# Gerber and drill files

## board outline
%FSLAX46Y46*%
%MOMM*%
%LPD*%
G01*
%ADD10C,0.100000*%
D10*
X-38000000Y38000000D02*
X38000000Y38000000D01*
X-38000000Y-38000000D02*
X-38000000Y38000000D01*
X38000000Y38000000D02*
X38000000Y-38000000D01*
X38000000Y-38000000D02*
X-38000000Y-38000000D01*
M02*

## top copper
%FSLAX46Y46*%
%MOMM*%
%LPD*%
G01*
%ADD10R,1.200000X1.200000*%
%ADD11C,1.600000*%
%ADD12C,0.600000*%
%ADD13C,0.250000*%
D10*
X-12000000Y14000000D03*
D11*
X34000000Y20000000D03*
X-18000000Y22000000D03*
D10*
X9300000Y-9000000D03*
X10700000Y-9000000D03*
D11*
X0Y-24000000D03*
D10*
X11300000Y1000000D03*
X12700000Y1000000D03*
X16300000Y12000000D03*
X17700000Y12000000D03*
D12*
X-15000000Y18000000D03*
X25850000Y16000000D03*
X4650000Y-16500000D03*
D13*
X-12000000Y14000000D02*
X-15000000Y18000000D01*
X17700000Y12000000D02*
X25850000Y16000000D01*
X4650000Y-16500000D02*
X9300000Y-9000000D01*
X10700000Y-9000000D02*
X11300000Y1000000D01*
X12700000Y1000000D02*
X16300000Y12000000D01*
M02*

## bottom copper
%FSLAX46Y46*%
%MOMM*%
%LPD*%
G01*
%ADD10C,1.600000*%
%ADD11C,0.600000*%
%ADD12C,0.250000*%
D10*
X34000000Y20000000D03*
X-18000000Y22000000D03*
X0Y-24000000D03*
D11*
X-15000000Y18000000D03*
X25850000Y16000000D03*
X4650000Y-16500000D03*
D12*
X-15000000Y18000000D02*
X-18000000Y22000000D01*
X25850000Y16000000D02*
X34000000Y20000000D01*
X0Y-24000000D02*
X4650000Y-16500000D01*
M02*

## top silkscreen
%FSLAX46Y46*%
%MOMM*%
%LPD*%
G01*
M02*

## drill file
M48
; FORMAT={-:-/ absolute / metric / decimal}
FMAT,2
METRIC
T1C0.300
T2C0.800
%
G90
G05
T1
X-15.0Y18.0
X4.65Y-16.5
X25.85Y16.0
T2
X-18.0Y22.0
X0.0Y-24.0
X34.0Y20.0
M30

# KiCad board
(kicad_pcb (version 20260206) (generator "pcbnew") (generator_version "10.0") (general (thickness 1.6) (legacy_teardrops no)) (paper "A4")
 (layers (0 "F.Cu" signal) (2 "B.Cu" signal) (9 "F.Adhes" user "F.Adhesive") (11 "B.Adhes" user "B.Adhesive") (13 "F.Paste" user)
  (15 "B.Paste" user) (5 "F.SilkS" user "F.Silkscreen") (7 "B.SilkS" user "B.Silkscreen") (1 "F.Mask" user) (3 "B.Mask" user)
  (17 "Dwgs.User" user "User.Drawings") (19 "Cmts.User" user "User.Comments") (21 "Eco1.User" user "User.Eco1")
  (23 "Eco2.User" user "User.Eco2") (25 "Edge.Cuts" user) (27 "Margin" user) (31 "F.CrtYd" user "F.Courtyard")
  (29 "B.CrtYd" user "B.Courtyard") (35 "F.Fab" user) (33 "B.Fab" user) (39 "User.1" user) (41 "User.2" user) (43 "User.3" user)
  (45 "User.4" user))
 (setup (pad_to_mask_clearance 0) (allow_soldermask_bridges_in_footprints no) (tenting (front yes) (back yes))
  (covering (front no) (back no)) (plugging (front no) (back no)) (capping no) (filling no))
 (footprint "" (layer "F.Cu") (at -12 -14)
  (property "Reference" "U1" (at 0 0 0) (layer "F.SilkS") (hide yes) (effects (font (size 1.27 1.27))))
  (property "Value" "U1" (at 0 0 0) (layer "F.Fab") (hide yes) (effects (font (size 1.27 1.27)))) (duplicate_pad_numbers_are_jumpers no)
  (pad "1" smd rect (at 0 0) (size 1.2 1.2) (layers "F.Cu" "F.Mask" "F.Paste") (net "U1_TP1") (thermal_bridge_angle 45)))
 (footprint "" (layer "F.Cu") (at 34 -20)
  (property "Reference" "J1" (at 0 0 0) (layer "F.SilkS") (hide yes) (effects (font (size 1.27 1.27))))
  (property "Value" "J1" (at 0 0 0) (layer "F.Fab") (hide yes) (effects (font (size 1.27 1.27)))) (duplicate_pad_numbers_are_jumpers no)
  (pad "1" thru_hole circle (at 0 0) (size 1.6 1.6) (drill 0.8) (layers "*.Cu" "*.Mask") (remove_unused_layers no) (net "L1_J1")))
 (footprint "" (layer "F.Cu") (at -18 -22)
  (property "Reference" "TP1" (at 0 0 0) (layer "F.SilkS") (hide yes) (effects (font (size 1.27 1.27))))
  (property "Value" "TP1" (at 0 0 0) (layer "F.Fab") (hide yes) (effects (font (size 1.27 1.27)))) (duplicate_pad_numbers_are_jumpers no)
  (pad "1" thru_hole circle (at 0 0) (size 1.6 1.6) (drill 0.8) (layers "*.Cu" "*.Mask") (remove_unused_layers no) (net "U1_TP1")))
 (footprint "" (layer "F.Cu") (at 10 9)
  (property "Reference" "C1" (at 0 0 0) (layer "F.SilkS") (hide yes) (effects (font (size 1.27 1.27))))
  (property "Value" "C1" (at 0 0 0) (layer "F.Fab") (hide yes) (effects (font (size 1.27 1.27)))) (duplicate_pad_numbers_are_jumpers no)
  (pad "1" smd rect (at -0.7 0) (size 1.2 1.2) (layers "F.Cu" "F.Mask" "F.Paste") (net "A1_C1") (thermal_bridge_angle 45))
  (pad "2" smd rect (at 0.7 0) (size 1.2 1.2) (layers "F.Cu" "F.Mask" "F.Paste") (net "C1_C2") (thermal_bridge_angle 45)))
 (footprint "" (layer "F.Cu") (at 0 24)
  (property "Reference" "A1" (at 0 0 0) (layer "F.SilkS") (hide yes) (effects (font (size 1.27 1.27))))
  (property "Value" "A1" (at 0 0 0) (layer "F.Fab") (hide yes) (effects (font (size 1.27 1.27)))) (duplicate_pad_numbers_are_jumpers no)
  (pad "1" thru_hole circle (at 0 0) (size 1.6 1.6) (drill 0.8) (layers "*.Cu" "*.Mask") (remove_unused_layers no) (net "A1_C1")))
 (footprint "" (layer "F.Cu") (at 12 -1)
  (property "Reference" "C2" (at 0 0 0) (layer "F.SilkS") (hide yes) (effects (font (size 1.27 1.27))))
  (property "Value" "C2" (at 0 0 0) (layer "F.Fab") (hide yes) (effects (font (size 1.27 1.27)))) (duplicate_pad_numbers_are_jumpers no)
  (pad "1" smd rect (at -0.7 0) (size 1.2 1.2) (layers "F.Cu" "F.Mask" "F.Paste") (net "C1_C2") (thermal_bridge_angle 45))
  (pad "2" smd rect (at 0.7 0) (size 1.2 1.2) (layers "F.Cu" "F.Mask" "F.Paste") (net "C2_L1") (thermal_bridge_angle 45)))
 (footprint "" (layer "F.Cu") (at 17 -12)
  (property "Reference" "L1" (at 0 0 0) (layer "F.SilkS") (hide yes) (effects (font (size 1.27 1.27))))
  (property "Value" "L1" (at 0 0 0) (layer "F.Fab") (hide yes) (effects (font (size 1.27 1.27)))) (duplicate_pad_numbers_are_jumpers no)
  (pad "1" smd rect (at -0.7 0) (size 1.2 1.2) (layers "F.Cu" "F.Mask" "F.Paste") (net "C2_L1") (thermal_bridge_angle 45))
  (pad "2" smd rect (at 0.7 0) (size 1.2 1.2) (layers "F.Cu" "F.Mask" "F.Paste") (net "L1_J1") (thermal_bridge_angle 45)))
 (gr_line (start -38 -38) (end 38 -38) (stroke (width 0.1) (type default)) (layer "Edge.Cuts"))
 (gr_line (start -38 38) (end -38 -38) (stroke (width 0.1) (type default)) (layer "Edge.Cuts"))
 (gr_line (start 38 -38) (end 38 38) (stroke (width 0.1) (type default)) (layer "Edge.Cuts"))
 (gr_line (start 38 38) (end -38 38) (stroke (width 0.1) (type default)) (layer "Edge.Cuts"))
 (segment (start -12 -14) (end -15 -18) (width 0.25) (layer "F.Cu") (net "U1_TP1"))
 (via (at -15 -18) (size 0.6) (drill 0.3) (layers "F.Cu" "B.Cu") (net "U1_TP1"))
 (segment (start -15 -18) (end -18 -22) (width 0.25) (layer "B.Cu") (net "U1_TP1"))
 (segment (start 17.7 -12) (end 25.85 -16) (width 0.25) (layer "F.Cu") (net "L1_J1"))
 (via (at 25.85 -16) (size 0.6) (drill 0.3) (layers "F.Cu" "B.Cu") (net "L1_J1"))
 (segment (start 25.85 -16) (end 34 -20) (width 0.25) (layer "B.Cu") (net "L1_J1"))
 (segment (start 4.65 16.5) (end 9.3 9) (width 0.25) (layer "F.Cu") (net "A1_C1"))
 (via (at 4.65 16.5) (size 0.6) (drill 0.3) (layers "F.Cu" "B.Cu") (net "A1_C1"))
 (segment (start 0 24) (end 4.65 16.5) (width 0.25) (layer "B.Cu") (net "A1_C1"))
 (segment (start 10.7 9) (end 11.3 -1) (width 0.25) (layer "F.Cu") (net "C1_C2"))
 (segment (start 12.7 -1) (end 16.3 -12) (width 0.25) (layer "F.Cu") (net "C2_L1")))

